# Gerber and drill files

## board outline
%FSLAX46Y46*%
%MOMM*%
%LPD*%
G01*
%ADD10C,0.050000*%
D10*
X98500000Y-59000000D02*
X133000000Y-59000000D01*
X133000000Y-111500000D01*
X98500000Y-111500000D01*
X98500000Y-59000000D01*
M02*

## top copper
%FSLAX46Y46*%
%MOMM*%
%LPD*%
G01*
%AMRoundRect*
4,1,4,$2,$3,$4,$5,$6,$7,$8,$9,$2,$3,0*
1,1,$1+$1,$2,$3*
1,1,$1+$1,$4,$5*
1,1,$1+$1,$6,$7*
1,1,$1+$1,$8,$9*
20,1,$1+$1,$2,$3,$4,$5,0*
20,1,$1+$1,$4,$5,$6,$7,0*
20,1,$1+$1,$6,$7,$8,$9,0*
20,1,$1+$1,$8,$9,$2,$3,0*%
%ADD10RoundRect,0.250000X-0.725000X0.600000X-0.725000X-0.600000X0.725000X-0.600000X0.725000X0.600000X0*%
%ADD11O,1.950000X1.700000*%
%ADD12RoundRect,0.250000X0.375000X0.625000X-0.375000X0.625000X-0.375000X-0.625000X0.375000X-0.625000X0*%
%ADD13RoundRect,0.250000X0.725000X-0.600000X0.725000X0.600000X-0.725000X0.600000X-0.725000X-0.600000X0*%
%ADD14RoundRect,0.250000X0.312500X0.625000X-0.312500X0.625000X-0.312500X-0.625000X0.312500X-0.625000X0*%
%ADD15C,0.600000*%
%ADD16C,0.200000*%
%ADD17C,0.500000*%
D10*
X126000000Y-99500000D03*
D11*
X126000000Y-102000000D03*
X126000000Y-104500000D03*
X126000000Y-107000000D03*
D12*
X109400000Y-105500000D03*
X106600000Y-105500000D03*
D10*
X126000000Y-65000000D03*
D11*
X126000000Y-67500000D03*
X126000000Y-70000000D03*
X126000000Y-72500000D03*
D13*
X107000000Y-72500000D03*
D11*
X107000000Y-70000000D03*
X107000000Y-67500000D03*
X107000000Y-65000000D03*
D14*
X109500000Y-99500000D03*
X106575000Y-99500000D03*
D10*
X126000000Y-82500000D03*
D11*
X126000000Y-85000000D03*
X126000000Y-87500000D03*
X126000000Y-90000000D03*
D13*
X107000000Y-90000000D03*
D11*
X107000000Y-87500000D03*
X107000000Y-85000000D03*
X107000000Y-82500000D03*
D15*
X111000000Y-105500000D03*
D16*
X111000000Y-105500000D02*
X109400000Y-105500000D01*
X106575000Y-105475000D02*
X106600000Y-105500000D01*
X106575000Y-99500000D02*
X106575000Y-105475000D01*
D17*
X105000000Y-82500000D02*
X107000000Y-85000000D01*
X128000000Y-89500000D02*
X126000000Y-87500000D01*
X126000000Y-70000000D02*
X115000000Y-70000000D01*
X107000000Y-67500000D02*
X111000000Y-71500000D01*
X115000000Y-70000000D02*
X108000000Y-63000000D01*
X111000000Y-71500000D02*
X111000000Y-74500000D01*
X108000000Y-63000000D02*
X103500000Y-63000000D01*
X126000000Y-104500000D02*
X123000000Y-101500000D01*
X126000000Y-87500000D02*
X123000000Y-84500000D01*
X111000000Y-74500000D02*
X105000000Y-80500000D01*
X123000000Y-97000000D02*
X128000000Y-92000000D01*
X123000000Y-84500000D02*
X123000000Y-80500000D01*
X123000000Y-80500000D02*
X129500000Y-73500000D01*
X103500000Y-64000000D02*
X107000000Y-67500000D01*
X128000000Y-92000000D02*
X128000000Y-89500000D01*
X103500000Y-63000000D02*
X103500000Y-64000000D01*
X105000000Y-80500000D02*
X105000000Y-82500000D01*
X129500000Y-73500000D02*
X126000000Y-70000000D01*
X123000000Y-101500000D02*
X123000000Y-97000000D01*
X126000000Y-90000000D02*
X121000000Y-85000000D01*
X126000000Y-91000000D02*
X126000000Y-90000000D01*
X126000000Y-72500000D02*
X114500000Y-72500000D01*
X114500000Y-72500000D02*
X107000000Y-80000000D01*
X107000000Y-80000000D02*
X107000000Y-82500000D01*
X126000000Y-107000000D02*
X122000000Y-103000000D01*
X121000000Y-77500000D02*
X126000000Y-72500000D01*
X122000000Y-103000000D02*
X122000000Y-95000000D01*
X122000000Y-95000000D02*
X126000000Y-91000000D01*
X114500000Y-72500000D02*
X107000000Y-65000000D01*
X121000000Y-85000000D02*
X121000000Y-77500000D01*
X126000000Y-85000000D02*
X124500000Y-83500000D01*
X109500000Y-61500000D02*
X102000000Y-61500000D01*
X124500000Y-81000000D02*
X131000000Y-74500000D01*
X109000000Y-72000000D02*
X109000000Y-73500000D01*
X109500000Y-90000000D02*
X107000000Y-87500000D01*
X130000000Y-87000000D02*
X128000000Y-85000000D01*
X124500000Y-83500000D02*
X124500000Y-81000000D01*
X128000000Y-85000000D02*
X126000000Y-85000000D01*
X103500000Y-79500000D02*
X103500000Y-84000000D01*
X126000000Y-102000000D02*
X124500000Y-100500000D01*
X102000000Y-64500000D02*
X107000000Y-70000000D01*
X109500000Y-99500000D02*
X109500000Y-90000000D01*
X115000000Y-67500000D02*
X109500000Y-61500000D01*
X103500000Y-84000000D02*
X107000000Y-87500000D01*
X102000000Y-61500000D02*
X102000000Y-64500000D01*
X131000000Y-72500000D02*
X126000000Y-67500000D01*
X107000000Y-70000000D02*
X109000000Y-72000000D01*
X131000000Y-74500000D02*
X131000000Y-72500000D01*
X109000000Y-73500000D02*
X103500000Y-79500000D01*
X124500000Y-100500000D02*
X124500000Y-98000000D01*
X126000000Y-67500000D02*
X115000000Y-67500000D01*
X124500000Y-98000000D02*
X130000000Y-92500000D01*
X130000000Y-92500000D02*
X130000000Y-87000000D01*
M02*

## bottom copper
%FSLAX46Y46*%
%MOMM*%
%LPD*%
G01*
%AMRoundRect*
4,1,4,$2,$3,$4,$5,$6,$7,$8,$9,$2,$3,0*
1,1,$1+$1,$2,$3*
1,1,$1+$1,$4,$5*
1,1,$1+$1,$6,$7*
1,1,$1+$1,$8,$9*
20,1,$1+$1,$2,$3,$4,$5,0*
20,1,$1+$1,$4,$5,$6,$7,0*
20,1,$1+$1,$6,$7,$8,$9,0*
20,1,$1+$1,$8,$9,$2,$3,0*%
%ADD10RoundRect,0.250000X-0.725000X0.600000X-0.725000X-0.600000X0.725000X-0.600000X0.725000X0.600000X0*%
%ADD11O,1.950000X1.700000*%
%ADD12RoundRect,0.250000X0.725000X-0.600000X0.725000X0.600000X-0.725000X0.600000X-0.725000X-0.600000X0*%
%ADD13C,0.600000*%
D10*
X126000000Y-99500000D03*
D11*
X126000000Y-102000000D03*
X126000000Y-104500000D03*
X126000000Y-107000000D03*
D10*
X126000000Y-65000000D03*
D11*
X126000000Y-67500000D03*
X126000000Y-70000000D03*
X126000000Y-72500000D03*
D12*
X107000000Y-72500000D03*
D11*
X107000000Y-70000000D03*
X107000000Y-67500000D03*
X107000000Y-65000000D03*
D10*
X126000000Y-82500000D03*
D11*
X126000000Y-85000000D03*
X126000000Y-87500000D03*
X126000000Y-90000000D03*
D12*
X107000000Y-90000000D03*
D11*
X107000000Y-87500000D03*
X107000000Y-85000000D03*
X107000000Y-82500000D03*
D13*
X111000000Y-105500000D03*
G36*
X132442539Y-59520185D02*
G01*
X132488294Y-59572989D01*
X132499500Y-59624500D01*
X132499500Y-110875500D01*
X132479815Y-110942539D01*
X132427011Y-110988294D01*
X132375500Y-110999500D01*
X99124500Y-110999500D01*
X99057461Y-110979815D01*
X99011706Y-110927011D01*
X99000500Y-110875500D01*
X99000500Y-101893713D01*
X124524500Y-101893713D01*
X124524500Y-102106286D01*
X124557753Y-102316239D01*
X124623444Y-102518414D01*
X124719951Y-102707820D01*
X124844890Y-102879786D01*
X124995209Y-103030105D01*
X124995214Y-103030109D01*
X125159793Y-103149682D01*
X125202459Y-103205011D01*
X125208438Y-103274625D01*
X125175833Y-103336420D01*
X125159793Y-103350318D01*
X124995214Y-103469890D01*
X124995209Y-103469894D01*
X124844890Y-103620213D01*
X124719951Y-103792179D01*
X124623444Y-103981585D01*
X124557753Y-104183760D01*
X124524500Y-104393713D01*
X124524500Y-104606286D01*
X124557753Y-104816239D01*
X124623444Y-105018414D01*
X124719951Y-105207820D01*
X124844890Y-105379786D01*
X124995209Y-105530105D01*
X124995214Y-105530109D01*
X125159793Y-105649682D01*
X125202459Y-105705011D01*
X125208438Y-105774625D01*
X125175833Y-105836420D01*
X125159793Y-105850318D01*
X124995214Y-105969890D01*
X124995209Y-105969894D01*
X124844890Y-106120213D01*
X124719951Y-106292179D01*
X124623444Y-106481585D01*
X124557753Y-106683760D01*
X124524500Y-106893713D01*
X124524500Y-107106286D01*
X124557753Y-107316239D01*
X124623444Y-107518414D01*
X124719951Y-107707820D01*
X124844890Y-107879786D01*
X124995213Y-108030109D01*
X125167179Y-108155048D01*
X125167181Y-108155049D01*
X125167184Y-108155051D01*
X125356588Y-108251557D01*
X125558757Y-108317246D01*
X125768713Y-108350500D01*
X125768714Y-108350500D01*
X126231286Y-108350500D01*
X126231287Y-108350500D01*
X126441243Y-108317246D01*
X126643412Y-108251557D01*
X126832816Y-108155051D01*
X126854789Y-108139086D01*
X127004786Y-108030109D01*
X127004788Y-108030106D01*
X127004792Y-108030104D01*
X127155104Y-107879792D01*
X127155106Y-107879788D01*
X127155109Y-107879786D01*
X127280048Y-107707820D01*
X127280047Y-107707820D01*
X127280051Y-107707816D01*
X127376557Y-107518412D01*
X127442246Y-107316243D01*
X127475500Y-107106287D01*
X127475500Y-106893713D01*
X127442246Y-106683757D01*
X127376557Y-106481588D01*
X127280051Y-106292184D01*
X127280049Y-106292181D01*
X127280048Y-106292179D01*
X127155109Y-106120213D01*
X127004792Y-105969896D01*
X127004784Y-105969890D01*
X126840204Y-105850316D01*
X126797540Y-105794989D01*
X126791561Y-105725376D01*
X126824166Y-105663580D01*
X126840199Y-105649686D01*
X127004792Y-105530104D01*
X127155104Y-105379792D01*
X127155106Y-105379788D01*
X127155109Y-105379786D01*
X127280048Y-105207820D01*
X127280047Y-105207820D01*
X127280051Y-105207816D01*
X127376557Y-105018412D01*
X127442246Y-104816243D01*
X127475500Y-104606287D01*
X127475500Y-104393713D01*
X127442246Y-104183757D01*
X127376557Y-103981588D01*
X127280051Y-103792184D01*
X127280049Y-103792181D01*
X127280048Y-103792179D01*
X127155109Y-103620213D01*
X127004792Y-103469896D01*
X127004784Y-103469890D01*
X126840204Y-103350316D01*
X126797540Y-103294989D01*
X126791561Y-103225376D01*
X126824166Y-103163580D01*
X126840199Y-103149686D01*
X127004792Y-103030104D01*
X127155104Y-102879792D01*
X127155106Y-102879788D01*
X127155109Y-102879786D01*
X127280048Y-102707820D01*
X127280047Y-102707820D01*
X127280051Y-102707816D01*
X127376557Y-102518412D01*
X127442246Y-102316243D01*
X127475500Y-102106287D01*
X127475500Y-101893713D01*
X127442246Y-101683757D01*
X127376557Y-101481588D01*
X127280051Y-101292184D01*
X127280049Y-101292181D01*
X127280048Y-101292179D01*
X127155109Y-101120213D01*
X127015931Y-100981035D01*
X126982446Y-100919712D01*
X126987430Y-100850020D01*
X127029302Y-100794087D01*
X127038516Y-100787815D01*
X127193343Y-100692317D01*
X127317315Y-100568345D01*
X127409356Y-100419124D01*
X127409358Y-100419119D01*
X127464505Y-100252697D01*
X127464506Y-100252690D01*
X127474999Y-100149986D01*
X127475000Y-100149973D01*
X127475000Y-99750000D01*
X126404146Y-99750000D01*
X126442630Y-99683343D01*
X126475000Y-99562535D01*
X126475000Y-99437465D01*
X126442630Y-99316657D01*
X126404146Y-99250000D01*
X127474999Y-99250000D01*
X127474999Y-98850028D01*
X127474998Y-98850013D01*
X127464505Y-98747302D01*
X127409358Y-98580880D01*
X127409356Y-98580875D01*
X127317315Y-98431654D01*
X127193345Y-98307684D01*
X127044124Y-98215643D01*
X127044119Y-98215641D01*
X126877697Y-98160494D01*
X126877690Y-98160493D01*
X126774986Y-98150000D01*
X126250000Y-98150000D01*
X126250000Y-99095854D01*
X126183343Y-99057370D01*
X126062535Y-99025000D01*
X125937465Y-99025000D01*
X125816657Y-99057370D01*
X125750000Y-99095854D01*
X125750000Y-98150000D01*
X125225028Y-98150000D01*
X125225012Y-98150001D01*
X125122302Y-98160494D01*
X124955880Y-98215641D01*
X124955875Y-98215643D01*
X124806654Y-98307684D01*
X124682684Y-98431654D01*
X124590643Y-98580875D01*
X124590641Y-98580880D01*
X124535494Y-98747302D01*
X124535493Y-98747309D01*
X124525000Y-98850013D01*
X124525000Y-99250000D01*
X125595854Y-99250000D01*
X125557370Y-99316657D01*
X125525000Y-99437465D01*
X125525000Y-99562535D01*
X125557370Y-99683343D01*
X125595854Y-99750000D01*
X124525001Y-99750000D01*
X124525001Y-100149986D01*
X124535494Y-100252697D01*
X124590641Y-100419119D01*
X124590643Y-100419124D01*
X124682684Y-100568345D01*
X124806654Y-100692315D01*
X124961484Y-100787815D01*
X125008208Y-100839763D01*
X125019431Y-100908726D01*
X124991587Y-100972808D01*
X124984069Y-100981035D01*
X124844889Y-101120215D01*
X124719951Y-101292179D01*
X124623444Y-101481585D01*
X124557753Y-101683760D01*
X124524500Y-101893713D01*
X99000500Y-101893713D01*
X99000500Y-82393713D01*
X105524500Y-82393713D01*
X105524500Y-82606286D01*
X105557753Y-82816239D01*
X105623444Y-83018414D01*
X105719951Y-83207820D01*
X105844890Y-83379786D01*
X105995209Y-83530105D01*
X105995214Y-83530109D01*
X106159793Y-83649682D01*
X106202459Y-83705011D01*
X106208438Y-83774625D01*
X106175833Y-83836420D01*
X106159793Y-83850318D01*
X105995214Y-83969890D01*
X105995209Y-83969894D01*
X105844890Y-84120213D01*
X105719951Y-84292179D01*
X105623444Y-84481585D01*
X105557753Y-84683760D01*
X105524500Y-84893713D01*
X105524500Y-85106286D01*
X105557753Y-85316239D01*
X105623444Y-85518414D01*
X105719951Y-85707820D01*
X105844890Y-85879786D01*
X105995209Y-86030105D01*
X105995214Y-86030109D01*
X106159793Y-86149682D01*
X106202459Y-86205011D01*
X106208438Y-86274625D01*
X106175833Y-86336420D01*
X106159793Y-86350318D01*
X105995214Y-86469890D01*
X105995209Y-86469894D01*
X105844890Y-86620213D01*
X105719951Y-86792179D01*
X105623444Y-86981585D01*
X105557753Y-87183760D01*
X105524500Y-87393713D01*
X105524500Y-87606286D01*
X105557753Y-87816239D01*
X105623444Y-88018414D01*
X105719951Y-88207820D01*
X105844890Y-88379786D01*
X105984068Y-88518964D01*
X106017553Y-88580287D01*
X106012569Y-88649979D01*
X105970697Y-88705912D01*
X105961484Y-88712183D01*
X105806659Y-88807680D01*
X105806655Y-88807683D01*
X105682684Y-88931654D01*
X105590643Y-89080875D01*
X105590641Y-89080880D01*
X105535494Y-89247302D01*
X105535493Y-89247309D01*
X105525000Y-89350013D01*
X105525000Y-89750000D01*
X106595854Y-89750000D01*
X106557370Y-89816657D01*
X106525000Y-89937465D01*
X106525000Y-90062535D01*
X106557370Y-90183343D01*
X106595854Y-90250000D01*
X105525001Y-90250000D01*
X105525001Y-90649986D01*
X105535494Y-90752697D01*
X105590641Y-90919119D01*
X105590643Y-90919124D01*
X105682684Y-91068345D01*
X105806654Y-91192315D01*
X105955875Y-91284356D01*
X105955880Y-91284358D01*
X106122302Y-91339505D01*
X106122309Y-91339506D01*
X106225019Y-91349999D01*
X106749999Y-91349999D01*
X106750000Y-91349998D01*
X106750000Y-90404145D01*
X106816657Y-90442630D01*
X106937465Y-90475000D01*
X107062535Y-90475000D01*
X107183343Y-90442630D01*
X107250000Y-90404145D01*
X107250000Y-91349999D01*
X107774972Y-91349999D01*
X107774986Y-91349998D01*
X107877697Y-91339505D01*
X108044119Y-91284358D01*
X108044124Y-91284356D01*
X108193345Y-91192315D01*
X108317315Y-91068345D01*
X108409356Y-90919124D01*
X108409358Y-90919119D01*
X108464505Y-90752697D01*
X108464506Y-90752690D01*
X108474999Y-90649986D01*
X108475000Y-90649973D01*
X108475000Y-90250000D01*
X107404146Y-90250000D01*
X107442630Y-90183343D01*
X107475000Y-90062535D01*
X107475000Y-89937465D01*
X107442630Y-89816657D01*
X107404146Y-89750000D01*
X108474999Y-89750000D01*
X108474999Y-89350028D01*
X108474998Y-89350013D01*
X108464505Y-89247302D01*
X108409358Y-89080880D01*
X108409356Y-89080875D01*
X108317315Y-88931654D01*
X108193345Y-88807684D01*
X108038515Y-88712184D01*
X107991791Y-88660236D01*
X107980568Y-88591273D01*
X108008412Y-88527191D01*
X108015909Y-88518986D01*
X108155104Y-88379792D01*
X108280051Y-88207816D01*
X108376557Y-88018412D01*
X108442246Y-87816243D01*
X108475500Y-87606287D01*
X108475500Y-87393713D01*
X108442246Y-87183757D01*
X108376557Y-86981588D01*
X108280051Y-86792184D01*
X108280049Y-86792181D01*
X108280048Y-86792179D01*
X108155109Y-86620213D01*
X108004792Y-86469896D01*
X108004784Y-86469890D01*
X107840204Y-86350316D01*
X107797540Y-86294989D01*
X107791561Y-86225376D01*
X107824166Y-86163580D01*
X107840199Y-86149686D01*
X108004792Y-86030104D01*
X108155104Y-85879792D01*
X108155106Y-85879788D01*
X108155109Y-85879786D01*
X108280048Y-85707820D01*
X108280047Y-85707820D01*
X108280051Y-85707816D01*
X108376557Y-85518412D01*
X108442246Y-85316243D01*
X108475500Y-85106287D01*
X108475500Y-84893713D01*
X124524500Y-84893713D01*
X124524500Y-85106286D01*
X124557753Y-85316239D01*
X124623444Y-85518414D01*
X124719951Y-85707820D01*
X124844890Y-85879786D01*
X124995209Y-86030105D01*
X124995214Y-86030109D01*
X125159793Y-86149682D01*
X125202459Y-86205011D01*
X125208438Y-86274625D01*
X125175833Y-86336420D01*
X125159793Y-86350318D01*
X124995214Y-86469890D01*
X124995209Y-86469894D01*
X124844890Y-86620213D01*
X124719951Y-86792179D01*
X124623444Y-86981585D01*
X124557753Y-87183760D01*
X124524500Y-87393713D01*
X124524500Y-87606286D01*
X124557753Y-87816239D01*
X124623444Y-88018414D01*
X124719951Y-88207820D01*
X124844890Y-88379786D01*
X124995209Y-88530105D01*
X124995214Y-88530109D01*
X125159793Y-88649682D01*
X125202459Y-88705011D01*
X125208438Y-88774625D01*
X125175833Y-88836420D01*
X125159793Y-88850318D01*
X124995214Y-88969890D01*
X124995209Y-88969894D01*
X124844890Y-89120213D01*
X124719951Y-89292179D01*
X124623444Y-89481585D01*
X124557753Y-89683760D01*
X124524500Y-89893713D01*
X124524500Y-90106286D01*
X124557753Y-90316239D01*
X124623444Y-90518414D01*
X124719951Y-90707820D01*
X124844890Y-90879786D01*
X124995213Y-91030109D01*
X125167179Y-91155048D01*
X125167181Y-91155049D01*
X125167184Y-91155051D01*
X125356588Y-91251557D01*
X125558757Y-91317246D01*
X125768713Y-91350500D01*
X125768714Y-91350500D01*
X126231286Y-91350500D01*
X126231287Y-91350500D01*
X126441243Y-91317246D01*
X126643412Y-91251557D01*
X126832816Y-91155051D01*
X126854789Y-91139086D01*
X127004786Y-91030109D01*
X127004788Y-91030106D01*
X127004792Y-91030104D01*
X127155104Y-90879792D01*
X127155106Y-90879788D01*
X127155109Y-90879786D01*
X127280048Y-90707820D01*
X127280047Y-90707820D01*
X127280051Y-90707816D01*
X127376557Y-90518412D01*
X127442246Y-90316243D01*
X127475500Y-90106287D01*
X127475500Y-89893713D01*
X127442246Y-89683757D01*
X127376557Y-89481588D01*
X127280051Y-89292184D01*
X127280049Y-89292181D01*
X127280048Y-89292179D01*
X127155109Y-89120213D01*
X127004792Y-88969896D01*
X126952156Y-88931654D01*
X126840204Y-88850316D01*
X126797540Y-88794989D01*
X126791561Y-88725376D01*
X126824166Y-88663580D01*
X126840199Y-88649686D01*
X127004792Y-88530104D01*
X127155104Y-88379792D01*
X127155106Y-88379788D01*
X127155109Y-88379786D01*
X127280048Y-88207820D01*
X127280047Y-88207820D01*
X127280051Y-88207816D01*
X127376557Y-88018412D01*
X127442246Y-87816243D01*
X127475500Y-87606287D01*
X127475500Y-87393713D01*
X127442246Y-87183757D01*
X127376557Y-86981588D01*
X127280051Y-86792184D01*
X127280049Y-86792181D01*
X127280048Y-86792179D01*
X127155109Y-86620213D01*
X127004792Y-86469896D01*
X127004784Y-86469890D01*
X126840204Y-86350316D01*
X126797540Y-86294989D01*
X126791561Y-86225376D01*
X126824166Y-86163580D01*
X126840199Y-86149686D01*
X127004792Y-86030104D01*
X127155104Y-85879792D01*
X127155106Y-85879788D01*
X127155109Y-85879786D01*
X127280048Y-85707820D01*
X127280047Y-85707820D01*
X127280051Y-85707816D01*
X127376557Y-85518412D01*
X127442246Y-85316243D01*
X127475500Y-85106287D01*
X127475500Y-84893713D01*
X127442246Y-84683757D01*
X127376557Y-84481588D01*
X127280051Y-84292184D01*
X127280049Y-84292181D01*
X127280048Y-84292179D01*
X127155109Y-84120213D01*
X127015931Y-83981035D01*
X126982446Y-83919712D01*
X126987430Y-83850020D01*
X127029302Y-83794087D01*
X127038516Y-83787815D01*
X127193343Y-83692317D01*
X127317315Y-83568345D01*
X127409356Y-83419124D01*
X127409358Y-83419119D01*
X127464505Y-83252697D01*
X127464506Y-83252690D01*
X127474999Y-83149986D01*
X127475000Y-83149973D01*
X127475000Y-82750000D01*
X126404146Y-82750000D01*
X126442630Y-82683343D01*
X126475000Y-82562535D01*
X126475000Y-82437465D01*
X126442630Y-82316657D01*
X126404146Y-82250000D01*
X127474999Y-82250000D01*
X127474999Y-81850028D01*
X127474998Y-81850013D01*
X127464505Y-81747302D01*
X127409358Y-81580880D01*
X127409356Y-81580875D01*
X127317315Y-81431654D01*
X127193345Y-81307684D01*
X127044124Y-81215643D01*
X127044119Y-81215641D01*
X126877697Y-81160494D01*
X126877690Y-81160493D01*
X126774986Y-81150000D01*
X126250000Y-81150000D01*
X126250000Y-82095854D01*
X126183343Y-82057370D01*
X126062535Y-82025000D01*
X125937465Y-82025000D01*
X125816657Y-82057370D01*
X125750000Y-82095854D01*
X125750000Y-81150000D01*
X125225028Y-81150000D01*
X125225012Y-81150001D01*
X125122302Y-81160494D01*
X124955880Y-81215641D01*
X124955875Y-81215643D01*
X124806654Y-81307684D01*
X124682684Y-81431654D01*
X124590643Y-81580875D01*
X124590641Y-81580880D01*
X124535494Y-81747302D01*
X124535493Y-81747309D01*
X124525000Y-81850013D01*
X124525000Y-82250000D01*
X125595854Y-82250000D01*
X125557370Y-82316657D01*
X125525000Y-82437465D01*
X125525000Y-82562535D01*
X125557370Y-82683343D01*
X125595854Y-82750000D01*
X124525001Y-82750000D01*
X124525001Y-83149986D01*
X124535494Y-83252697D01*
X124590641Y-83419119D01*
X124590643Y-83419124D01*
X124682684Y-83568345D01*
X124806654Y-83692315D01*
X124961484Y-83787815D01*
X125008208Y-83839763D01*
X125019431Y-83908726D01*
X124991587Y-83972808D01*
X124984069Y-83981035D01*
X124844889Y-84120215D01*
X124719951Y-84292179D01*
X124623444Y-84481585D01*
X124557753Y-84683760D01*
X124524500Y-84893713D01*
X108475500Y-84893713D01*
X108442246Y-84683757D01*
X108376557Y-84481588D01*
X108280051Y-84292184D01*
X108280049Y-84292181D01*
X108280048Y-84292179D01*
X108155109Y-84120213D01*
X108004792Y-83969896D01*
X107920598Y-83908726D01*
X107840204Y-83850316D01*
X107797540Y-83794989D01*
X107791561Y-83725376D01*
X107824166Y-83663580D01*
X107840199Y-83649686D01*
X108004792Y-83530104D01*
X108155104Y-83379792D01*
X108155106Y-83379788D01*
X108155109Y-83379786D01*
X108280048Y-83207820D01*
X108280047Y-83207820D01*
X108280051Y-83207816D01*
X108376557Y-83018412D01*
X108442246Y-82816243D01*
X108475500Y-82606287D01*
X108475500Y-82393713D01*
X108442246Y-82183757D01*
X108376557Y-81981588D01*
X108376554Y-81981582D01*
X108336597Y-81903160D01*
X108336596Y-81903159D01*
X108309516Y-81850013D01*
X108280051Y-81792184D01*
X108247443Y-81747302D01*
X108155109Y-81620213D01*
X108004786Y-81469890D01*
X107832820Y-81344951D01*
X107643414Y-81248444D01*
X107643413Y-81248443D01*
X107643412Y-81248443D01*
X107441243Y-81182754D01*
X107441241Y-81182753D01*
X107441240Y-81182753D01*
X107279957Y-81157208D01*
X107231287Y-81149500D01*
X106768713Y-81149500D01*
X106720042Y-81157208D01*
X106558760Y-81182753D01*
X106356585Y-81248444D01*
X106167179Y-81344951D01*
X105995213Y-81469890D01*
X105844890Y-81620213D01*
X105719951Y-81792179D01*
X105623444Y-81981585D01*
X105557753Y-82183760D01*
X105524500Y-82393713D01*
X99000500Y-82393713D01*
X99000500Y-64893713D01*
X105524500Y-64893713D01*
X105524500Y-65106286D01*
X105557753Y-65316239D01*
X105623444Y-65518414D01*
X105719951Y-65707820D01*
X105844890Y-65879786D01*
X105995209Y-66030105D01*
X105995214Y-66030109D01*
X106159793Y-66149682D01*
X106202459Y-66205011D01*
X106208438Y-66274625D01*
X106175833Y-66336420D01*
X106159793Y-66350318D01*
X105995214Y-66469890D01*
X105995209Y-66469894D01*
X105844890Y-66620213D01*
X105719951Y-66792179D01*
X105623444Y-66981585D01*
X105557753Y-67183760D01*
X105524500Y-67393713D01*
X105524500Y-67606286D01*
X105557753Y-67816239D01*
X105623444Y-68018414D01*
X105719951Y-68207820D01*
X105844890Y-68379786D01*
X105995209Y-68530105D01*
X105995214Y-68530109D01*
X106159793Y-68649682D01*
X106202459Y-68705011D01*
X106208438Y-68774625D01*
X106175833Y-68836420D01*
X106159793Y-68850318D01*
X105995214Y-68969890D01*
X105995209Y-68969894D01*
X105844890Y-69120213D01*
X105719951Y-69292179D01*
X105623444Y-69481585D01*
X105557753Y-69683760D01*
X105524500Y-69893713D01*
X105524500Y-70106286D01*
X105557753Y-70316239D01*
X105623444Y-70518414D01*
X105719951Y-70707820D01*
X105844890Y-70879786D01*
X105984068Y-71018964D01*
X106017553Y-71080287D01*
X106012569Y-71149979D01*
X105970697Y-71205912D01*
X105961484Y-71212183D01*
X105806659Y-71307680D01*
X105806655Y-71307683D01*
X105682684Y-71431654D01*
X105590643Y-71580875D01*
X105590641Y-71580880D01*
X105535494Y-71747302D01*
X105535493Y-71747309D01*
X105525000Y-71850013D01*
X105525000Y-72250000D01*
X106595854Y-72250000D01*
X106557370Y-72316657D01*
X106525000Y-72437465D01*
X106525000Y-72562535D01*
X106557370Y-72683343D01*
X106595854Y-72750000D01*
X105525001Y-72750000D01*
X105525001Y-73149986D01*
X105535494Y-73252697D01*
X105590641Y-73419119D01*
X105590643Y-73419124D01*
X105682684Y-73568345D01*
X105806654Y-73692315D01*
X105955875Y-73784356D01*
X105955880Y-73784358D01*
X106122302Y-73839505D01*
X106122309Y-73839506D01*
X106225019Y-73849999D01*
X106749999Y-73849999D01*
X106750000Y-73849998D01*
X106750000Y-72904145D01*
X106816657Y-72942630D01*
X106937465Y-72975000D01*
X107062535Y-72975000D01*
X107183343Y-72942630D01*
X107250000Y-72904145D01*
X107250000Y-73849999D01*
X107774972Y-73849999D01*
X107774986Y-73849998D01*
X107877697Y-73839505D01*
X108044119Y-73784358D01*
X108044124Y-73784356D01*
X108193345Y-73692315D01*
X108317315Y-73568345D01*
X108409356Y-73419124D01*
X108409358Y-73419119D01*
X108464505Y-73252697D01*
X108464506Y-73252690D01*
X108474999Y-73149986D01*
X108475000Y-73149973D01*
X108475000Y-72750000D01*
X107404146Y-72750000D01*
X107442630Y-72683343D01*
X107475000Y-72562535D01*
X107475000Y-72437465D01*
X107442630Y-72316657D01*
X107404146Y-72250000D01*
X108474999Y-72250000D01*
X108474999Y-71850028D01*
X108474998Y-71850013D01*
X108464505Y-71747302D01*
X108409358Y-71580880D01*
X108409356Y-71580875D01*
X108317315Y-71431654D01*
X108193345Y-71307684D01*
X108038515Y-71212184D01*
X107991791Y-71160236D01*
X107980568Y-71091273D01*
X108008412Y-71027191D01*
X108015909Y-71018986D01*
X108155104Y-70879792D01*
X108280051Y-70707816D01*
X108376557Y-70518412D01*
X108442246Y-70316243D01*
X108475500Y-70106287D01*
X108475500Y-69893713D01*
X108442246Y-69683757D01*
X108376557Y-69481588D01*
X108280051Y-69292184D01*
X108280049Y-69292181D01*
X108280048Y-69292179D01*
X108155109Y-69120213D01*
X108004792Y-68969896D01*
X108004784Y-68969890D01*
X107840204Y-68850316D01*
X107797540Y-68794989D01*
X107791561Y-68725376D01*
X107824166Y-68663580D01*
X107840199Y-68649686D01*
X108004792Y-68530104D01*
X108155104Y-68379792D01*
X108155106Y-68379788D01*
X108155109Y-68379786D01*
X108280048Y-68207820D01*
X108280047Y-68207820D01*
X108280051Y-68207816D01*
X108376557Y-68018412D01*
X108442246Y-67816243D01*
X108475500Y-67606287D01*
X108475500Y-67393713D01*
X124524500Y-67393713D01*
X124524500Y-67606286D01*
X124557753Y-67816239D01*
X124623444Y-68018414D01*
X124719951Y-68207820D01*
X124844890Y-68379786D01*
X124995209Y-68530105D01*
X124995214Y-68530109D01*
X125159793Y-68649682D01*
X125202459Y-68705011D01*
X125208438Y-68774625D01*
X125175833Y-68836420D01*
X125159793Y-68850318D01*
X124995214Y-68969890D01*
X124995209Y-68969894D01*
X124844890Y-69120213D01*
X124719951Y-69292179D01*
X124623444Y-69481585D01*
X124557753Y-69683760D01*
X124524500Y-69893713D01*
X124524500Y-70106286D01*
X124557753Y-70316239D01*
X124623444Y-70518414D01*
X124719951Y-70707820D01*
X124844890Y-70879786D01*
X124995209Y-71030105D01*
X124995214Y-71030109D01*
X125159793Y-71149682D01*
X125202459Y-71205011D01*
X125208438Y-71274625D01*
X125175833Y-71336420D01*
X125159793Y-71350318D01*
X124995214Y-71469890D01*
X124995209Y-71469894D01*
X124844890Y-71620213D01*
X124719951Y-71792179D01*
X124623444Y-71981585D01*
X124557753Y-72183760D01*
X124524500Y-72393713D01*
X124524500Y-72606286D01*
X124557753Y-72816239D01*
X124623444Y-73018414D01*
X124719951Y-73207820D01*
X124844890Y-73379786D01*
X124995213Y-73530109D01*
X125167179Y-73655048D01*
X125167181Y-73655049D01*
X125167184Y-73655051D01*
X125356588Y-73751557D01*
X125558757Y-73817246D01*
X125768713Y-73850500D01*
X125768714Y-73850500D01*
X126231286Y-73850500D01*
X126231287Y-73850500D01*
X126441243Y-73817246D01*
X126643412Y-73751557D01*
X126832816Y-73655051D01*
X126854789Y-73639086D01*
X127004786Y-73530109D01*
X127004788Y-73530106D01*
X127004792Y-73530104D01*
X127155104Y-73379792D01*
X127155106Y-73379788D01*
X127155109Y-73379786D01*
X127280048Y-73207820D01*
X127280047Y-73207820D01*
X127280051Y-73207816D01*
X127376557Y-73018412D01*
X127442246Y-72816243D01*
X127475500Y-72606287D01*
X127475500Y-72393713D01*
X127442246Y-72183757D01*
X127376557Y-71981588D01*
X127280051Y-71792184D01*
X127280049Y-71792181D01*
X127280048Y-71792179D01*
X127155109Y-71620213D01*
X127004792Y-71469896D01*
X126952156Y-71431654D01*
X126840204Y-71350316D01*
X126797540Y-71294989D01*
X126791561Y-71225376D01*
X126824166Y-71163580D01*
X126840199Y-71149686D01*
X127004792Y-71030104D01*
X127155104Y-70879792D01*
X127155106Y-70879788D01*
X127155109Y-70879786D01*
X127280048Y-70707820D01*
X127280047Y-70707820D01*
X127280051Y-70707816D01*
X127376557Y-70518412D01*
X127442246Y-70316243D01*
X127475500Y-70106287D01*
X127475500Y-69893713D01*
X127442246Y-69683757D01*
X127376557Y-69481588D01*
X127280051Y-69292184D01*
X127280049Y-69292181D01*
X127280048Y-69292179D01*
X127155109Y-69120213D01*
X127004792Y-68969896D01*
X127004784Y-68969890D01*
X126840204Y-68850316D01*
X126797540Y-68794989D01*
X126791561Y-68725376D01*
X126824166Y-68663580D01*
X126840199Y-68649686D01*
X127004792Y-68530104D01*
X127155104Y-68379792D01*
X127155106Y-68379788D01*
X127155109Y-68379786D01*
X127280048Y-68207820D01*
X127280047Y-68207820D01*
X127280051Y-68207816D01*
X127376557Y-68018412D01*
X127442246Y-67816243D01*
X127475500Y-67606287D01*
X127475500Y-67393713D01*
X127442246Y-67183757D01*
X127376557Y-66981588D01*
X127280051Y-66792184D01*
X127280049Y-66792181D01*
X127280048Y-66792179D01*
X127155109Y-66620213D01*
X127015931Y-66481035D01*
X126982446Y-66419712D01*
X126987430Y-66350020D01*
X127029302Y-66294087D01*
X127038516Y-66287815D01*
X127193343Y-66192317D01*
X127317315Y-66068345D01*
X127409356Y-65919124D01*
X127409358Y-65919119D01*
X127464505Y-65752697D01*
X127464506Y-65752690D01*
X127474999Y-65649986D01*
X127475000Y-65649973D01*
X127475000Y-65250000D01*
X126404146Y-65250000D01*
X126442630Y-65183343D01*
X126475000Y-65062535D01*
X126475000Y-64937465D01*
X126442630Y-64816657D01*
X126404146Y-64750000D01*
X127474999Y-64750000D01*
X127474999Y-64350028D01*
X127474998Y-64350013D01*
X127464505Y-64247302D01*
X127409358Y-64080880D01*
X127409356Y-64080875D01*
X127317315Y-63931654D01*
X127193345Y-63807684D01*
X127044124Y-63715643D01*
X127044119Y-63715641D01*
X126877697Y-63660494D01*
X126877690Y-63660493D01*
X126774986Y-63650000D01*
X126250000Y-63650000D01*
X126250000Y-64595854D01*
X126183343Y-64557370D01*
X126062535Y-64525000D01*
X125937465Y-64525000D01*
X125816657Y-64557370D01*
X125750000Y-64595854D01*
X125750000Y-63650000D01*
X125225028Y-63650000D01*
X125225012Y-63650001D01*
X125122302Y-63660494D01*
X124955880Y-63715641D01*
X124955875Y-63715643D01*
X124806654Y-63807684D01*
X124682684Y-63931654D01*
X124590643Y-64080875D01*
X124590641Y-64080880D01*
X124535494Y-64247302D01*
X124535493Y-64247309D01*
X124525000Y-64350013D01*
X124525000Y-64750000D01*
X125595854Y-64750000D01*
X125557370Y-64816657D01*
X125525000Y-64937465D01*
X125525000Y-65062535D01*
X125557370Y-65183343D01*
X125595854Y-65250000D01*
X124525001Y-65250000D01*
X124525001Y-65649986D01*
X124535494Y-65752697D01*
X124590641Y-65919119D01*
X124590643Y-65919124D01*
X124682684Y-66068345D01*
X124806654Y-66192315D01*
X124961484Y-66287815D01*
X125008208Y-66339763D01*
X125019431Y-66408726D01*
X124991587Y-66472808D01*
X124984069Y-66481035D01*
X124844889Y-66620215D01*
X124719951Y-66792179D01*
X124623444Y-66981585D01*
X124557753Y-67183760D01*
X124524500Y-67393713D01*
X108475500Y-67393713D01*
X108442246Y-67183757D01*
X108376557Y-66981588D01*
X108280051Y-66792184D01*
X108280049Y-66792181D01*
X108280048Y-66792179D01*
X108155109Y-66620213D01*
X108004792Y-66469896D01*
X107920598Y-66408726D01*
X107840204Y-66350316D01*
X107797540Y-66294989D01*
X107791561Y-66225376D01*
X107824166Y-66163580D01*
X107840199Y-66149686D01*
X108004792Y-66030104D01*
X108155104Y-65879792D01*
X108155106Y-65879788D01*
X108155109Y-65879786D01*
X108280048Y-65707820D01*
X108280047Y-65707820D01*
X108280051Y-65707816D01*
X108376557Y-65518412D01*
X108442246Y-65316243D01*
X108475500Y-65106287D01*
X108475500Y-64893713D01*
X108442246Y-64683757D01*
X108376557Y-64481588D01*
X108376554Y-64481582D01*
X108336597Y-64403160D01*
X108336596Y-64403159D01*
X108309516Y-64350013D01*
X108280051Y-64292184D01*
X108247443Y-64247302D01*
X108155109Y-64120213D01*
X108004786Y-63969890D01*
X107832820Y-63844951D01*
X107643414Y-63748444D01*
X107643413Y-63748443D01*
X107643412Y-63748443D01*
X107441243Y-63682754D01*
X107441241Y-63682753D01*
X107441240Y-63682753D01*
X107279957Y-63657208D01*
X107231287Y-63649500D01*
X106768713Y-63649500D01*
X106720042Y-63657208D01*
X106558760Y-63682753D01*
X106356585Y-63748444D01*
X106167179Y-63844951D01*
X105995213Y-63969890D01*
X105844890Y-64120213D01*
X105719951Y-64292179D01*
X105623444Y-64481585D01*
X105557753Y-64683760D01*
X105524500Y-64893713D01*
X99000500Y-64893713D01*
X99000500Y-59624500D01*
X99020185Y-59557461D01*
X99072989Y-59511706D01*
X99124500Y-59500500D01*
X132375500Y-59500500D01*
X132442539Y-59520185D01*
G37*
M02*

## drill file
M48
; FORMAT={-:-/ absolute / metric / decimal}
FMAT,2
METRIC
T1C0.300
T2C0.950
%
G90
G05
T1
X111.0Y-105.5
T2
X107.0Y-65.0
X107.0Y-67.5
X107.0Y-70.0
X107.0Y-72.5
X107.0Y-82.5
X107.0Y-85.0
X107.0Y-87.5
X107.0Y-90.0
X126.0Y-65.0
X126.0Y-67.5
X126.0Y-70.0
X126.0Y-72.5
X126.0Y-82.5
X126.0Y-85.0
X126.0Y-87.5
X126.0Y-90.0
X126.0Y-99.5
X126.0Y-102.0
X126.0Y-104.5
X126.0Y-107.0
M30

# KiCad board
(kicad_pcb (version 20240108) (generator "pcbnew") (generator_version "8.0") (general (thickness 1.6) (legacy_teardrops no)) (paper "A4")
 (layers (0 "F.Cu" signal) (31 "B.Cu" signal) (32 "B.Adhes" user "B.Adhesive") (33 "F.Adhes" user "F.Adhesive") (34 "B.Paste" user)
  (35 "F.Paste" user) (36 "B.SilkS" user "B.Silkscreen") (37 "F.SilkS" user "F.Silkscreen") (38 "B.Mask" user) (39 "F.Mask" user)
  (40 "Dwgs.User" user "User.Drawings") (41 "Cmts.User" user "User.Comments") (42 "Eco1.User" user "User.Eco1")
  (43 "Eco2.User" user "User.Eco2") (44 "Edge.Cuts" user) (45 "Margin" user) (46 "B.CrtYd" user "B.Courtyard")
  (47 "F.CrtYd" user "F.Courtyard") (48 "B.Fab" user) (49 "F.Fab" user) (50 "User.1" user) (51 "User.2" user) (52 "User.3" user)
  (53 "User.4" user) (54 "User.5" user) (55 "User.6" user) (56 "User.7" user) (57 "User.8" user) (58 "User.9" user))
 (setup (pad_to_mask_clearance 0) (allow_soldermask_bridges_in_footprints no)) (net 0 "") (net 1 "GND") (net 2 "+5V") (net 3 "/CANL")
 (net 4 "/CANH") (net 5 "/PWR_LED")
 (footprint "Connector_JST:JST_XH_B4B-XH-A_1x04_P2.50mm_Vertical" (layer "F.Cu") (at 126 99.5 -90)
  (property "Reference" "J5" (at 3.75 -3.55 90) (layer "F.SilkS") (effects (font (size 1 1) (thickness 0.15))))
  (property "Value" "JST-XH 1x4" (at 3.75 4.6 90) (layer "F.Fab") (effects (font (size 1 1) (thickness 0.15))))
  (pad "1" thru_hole roundrect (at 0 0 270) (size 1.7 1.95) (drill 0.95) (layers "*.Cu" "*.Mask") (remove_unused_layers no)
   (roundrect_rratio 0.147059) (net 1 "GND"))
  (pad "2" thru_hole oval (at 2.5 0 270) (size 1.7 1.95) (drill 0.95) (layers "*.Cu" "*.Mask") (remove_unused_layers no) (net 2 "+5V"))
  (pad "3" thru_hole oval (at 5 0 270) (size 1.7 1.95) (drill 0.95) (layers "*.Cu" "*.Mask") (remove_unused_layers no) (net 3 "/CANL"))
  (pad "4" thru_hole oval (at 7.5 0 270) (size 1.7 1.95) (drill 0.95) (layers "*.Cu" "*.Mask") (remove_unused_layers no) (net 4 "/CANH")))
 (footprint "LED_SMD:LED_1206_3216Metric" (layer "F.Cu") (at 108 105.5 180)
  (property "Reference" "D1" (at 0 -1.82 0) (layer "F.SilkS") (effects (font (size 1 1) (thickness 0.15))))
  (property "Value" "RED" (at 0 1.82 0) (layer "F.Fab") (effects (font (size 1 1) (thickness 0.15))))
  (pad "1" smd roundrect (at -1.4 0 180) (size 1.25 1.75) (layers "F.Cu" "F.Paste" "F.Mask") (roundrect_rratio 0.2) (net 1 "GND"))
  (pad "2" smd roundrect (at 1.4 0 180) (size 1.25 1.75) (layers "F.Cu" "F.Paste" "F.Mask") (roundrect_rratio 0.2) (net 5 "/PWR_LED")))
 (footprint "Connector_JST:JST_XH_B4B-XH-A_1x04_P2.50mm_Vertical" (layer "F.Cu") (at 126 65 -90)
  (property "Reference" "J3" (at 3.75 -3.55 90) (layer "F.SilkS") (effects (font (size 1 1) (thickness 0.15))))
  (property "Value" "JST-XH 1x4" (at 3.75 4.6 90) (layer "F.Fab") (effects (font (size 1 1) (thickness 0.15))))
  (pad "1" thru_hole roundrect (at 0 0 270) (size 1.7 1.95) (drill 0.95) (layers "*.Cu" "*.Mask") (remove_unused_layers no)
   (roundrect_rratio 0.147059) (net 1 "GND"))
  (pad "2" thru_hole oval (at 2.5 0 270) (size 1.7 1.95) (drill 0.95) (layers "*.Cu" "*.Mask") (remove_unused_layers no) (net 2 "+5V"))
  (pad "3" thru_hole oval (at 5 0 270) (size 1.7 1.95) (drill 0.95) (layers "*.Cu" "*.Mask") (remove_unused_layers no) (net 3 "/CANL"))
  (pad "4" thru_hole oval (at 7.5 0 270) (size 1.7 1.95) (drill 0.95) (layers "*.Cu" "*.Mask") (remove_unused_layers no) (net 4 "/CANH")))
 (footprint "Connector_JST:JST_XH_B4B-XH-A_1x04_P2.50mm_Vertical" (layer "F.Cu") (at 107 72.5 90)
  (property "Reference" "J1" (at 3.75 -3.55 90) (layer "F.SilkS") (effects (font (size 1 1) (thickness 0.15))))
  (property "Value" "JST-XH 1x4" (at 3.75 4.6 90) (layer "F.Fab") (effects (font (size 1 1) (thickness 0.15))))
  (pad "1" thru_hole roundrect (at 0 0 90) (size 1.7 1.95) (drill 0.95) (layers "*.Cu" "*.Mask") (remove_unused_layers no)
   (roundrect_rratio 0.147059) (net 1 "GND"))
  (pad "2" thru_hole oval (at 2.5 0 90) (size 1.7 1.95) (drill 0.95) (layers "*.Cu" "*.Mask") (remove_unused_layers no) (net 2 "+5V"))
  (pad "3" thru_hole oval (at 5 0 90) (size 1.7 1.95) (drill 0.95) (layers "*.Cu" "*.Mask") (remove_unused_layers no) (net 3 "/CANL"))
  (pad "4" thru_hole oval (at 7.5 0 90) (size 1.7 1.95) (drill 0.95) (layers "*.Cu" "*.Mask") (remove_unused_layers no) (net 4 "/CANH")))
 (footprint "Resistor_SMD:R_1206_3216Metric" (layer "F.Cu") (at 108.0375 99.5 180)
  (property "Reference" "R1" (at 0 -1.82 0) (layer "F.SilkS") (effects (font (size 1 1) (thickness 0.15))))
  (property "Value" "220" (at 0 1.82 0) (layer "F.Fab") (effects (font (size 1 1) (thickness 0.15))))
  (pad "1" smd roundrect (at -1.4625 0 180) (size 1.125 1.75) (layers "F.Cu" "F.Paste" "F.Mask") (roundrect_rratio 0.222222) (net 2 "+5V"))
  (pad "2" smd roundrect (at 1.4625 0 180) (size 1.125 1.75) (layers "F.Cu" "F.Paste" "F.Mask") (roundrect_rratio 0.222222)
   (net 5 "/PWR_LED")))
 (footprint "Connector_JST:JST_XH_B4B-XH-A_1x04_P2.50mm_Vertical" (layer "F.Cu") (at 126 82.5 -90)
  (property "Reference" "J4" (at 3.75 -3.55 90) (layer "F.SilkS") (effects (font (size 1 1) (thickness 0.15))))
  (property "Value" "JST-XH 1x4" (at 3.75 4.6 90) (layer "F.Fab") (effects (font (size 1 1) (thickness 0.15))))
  (pad "1" thru_hole roundrect (at 0 0 270) (size 1.7 1.95) (drill 0.95) (layers "*.Cu" "*.Mask") (remove_unused_layers no)
   (roundrect_rratio 0.147059) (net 1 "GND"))
  (pad "2" thru_hole oval (at 2.5 0 270) (size 1.7 1.95) (drill 0.95) (layers "*.Cu" "*.Mask") (remove_unused_layers no) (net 2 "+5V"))
  (pad "3" thru_hole oval (at 5 0 270) (size 1.7 1.95) (drill 0.95) (layers "*.Cu" "*.Mask") (remove_unused_layers no) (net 3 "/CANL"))
  (pad "4" thru_hole oval (at 7.5 0 270) (size 1.7 1.95) (drill 0.95) (layers "*.Cu" "*.Mask") (remove_unused_layers no) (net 4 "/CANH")))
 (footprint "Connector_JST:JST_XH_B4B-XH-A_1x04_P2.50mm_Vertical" (layer "F.Cu") (at 107 90 90)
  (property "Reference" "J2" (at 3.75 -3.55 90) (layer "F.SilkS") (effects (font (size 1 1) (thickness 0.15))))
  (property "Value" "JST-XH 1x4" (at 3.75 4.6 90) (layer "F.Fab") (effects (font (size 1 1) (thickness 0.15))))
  (pad "1" thru_hole roundrect (at 0 0 90) (size 1.7 1.95) (drill 0.95) (layers "*.Cu" "*.Mask") (remove_unused_layers no)
   (roundrect_rratio 0.147059) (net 1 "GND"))
  (pad "2" thru_hole oval (at 2.5 0 90) (size 1.7 1.95) (drill 0.95) (layers "*.Cu" "*.Mask") (remove_unused_layers no) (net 2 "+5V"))
  (pad "3" thru_hole oval (at 5 0 90) (size 1.7 1.95) (drill 0.95) (layers "*.Cu" "*.Mask") (remove_unused_layers no) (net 3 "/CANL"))
  (pad "4" thru_hole oval (at 7.5 0 90) (size 1.7 1.95) (drill 0.95) (layers "*.Cu" "*.Mask") (remove_unused_layers no) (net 4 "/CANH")))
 (gr_rect (start 98.5 59) (end 133 111.5) (stroke (width 0.05) (type default)) (fill none) (layer "Edge.Cuts"))
 (segment (start 111 105.5) (end 109.4 105.5) (width 0.2) (layer "F.Cu") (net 1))
 (via (at 111 105.5) (size 0.6) (drill 0.3) (layers "F.Cu" "B.Cu") (free yes) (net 1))
 (segment (start 106.575 105.475) (end 106.6 105.5) (width 0.2) (layer "F.Cu") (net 5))
 (segment (start 106.575 99.5) (end 106.575 105.475) (width 0.2) (layer "F.Cu") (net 5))
 (segment (start 105 82.5) (end 107 85) (width 0.5) (layer "F.Cu") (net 3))
 (segment (start 128 89.5) (end 126 87.5) (width 0.5) (layer "F.Cu") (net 3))
 (segment (start 126 70) (end 115 70) (width 0.5) (layer "F.Cu") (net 3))
 (segment (start 107 67.5) (end 111 71.5) (width 0.5) (layer "F.Cu") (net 3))
 (segment (start 115 70) (end 108 63) (width 0.5) (layer "F.Cu") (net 3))
 (segment (start 111 71.5) (end 111 74.5) (width 0.5) (layer "F.Cu") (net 3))
 (segment (start 108 63) (end 103.5 63) (width 0.5) (layer "F.Cu") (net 3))
 (segment (start 126 104.5) (end 123 101.5) (width 0.5) (layer "F.Cu") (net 3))
 (segment (start 126 87.5) (end 123 84.5) (width 0.5) (layer "F.Cu") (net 3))
 (segment (start 111 74.5) (end 105 80.5) (width 0.5) (layer "F.Cu") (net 3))
 (segment (start 123 97) (end 128 92) (width 0.5) (layer "F.Cu") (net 3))
 (segment (start 123 84.5) (end 123 80.5) (width 0.5) (layer "F.Cu") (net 3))
 (segment (start 123 80.5) (end 129.5 73.5) (width 0.5) (layer "F.Cu") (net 3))
 (segment (start 103.5 64) (end 107 67.5) (width 0.5) (layer "F.Cu") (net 3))
 (segment (start 128 92) (end 128 89.5) (width 0.5) (layer "F.Cu") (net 3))
 (segment (start 103.5 63) (end 103.5 64) (width 0.5) (layer "F.Cu") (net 3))
 (segment (start 105 80.5) (end 105 82.5) (width 0.5) (layer "F.Cu") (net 3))
 (segment (start 129.5 73.5) (end 126 70) (width 0.5) (layer "F.Cu") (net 3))
 (segment (start 123 101.5) (end 123 97) (width 0.5) (layer "F.Cu") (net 3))
 (segment (start 126 90) (end 121 85) (width 0.5) (layer "F.Cu") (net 4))
 (segment (start 126 91) (end 126 90) (width 0.5) (layer "F.Cu") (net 4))
 (segment (start 126 72.5) (end 114.5 72.5) (width 0.5) (layer "F.Cu") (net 4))
 (segment (start 114.5 72.5) (end 107 80) (width 0.5) (layer "F.Cu") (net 4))
 (segment (start 107 80) (end 107 82.5) (width 0.5) (layer "F.Cu") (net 4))
 (segment (start 126 107) (end 122 103) (width 0.5) (layer "F.Cu") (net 4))
 (segment (start 121 77.5) (end 126 72.5) (width 0.5) (layer "F.Cu") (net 4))
 (segment (start 122 103) (end 122 95) (width 0.5) (layer "F.Cu") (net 4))
 (segment (start 122 95) (end 126 91) (width 0.5) (layer "F.Cu") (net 4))
 (segment (start 114.5 72.5) (end 107 65) (width 0.5) (layer "F.Cu") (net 4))
 (segment (start 121 85) (end 121 77.5) (width 0.5) (layer "F.Cu") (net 4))
 (segment (start 126 85) (end 124.5 83.5) (width 0.5) (layer "F.Cu") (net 2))
 (segment (start 109.5 61.5) (end 102 61.5) (width 0.5) (layer "F.Cu") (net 2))
 (segment (start 124.5 81) (end 131 74.5) (width 0.5) (layer "F.Cu") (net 2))
 (segment (start 109 72) (end 109 73.5) (width 0.5) (layer "F.Cu") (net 2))
 (segment (start 109.5 90) (end 107 87.5) (width 0.5) (layer "F.Cu") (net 2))
 (segment (start 130 87) (end 128 85) (width 0.5) (layer "F.Cu") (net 2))
 (segment (start 124.5 83.5) (end 124.5 81) (width 0.5) (layer "F.Cu") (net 2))
 (segment (start 128 85) (end 126 85) (width 0.5) (layer "F.Cu") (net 2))
 (segment (start 103.5 79.5) (end 103.5 84) (width 0.5) (layer "F.Cu") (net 2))
 (segment (start 126 102) (end 124.5 100.5) (width 0.5) (layer "F.Cu") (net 2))
 (segment (start 102 64.5) (end 107 70) (width 0.5) (layer "F.Cu") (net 2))
 (segment (start 109.5 99.5) (end 109.5 90) (width 0.5) (layer "F.Cu") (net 2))
 (segment (start 115 67.5) (end 109.5 61.5) (width 0.5) (layer "F.Cu") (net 2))
 (segment (start 103.5 84) (end 107 87.5) (width 0.5) (layer "F.Cu") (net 2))
 (segment (start 102 61.5) (end 102 64.5) (width 0.5) (layer "F.Cu") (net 2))
 (segment (start 131 72.5) (end 126 67.5) (width 0.5) (layer "F.Cu") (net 2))
 (segment (start 107 70) (end 109 72) (width 0.5) (layer "F.Cu") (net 2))
 (segment (start 131 74.5) (end 131 72.5) (width 0.5) (layer "F.Cu") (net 2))
 (segment (start 109 73.5) (end 103.5 79.5) (width 0.5) (layer "F.Cu") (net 2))
 (segment (start 124.5 100.5) (end 124.5 98) (width 0.5) (layer "F.Cu") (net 2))
 (segment (start 126 67.5) (end 115 67.5) (width 0.5) (layer "F.Cu") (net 2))
 (segment (start 124.5 98) (end 130 92.5) (width 0.5) (layer "F.Cu") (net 2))
 (segment (start 130 92.5) (end 130 87) (width 0.5) (layer "F.Cu") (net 2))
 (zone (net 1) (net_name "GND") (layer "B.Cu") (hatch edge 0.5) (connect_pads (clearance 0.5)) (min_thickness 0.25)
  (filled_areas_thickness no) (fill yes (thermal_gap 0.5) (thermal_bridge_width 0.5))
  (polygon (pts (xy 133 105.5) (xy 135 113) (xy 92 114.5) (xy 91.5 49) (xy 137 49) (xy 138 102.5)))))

